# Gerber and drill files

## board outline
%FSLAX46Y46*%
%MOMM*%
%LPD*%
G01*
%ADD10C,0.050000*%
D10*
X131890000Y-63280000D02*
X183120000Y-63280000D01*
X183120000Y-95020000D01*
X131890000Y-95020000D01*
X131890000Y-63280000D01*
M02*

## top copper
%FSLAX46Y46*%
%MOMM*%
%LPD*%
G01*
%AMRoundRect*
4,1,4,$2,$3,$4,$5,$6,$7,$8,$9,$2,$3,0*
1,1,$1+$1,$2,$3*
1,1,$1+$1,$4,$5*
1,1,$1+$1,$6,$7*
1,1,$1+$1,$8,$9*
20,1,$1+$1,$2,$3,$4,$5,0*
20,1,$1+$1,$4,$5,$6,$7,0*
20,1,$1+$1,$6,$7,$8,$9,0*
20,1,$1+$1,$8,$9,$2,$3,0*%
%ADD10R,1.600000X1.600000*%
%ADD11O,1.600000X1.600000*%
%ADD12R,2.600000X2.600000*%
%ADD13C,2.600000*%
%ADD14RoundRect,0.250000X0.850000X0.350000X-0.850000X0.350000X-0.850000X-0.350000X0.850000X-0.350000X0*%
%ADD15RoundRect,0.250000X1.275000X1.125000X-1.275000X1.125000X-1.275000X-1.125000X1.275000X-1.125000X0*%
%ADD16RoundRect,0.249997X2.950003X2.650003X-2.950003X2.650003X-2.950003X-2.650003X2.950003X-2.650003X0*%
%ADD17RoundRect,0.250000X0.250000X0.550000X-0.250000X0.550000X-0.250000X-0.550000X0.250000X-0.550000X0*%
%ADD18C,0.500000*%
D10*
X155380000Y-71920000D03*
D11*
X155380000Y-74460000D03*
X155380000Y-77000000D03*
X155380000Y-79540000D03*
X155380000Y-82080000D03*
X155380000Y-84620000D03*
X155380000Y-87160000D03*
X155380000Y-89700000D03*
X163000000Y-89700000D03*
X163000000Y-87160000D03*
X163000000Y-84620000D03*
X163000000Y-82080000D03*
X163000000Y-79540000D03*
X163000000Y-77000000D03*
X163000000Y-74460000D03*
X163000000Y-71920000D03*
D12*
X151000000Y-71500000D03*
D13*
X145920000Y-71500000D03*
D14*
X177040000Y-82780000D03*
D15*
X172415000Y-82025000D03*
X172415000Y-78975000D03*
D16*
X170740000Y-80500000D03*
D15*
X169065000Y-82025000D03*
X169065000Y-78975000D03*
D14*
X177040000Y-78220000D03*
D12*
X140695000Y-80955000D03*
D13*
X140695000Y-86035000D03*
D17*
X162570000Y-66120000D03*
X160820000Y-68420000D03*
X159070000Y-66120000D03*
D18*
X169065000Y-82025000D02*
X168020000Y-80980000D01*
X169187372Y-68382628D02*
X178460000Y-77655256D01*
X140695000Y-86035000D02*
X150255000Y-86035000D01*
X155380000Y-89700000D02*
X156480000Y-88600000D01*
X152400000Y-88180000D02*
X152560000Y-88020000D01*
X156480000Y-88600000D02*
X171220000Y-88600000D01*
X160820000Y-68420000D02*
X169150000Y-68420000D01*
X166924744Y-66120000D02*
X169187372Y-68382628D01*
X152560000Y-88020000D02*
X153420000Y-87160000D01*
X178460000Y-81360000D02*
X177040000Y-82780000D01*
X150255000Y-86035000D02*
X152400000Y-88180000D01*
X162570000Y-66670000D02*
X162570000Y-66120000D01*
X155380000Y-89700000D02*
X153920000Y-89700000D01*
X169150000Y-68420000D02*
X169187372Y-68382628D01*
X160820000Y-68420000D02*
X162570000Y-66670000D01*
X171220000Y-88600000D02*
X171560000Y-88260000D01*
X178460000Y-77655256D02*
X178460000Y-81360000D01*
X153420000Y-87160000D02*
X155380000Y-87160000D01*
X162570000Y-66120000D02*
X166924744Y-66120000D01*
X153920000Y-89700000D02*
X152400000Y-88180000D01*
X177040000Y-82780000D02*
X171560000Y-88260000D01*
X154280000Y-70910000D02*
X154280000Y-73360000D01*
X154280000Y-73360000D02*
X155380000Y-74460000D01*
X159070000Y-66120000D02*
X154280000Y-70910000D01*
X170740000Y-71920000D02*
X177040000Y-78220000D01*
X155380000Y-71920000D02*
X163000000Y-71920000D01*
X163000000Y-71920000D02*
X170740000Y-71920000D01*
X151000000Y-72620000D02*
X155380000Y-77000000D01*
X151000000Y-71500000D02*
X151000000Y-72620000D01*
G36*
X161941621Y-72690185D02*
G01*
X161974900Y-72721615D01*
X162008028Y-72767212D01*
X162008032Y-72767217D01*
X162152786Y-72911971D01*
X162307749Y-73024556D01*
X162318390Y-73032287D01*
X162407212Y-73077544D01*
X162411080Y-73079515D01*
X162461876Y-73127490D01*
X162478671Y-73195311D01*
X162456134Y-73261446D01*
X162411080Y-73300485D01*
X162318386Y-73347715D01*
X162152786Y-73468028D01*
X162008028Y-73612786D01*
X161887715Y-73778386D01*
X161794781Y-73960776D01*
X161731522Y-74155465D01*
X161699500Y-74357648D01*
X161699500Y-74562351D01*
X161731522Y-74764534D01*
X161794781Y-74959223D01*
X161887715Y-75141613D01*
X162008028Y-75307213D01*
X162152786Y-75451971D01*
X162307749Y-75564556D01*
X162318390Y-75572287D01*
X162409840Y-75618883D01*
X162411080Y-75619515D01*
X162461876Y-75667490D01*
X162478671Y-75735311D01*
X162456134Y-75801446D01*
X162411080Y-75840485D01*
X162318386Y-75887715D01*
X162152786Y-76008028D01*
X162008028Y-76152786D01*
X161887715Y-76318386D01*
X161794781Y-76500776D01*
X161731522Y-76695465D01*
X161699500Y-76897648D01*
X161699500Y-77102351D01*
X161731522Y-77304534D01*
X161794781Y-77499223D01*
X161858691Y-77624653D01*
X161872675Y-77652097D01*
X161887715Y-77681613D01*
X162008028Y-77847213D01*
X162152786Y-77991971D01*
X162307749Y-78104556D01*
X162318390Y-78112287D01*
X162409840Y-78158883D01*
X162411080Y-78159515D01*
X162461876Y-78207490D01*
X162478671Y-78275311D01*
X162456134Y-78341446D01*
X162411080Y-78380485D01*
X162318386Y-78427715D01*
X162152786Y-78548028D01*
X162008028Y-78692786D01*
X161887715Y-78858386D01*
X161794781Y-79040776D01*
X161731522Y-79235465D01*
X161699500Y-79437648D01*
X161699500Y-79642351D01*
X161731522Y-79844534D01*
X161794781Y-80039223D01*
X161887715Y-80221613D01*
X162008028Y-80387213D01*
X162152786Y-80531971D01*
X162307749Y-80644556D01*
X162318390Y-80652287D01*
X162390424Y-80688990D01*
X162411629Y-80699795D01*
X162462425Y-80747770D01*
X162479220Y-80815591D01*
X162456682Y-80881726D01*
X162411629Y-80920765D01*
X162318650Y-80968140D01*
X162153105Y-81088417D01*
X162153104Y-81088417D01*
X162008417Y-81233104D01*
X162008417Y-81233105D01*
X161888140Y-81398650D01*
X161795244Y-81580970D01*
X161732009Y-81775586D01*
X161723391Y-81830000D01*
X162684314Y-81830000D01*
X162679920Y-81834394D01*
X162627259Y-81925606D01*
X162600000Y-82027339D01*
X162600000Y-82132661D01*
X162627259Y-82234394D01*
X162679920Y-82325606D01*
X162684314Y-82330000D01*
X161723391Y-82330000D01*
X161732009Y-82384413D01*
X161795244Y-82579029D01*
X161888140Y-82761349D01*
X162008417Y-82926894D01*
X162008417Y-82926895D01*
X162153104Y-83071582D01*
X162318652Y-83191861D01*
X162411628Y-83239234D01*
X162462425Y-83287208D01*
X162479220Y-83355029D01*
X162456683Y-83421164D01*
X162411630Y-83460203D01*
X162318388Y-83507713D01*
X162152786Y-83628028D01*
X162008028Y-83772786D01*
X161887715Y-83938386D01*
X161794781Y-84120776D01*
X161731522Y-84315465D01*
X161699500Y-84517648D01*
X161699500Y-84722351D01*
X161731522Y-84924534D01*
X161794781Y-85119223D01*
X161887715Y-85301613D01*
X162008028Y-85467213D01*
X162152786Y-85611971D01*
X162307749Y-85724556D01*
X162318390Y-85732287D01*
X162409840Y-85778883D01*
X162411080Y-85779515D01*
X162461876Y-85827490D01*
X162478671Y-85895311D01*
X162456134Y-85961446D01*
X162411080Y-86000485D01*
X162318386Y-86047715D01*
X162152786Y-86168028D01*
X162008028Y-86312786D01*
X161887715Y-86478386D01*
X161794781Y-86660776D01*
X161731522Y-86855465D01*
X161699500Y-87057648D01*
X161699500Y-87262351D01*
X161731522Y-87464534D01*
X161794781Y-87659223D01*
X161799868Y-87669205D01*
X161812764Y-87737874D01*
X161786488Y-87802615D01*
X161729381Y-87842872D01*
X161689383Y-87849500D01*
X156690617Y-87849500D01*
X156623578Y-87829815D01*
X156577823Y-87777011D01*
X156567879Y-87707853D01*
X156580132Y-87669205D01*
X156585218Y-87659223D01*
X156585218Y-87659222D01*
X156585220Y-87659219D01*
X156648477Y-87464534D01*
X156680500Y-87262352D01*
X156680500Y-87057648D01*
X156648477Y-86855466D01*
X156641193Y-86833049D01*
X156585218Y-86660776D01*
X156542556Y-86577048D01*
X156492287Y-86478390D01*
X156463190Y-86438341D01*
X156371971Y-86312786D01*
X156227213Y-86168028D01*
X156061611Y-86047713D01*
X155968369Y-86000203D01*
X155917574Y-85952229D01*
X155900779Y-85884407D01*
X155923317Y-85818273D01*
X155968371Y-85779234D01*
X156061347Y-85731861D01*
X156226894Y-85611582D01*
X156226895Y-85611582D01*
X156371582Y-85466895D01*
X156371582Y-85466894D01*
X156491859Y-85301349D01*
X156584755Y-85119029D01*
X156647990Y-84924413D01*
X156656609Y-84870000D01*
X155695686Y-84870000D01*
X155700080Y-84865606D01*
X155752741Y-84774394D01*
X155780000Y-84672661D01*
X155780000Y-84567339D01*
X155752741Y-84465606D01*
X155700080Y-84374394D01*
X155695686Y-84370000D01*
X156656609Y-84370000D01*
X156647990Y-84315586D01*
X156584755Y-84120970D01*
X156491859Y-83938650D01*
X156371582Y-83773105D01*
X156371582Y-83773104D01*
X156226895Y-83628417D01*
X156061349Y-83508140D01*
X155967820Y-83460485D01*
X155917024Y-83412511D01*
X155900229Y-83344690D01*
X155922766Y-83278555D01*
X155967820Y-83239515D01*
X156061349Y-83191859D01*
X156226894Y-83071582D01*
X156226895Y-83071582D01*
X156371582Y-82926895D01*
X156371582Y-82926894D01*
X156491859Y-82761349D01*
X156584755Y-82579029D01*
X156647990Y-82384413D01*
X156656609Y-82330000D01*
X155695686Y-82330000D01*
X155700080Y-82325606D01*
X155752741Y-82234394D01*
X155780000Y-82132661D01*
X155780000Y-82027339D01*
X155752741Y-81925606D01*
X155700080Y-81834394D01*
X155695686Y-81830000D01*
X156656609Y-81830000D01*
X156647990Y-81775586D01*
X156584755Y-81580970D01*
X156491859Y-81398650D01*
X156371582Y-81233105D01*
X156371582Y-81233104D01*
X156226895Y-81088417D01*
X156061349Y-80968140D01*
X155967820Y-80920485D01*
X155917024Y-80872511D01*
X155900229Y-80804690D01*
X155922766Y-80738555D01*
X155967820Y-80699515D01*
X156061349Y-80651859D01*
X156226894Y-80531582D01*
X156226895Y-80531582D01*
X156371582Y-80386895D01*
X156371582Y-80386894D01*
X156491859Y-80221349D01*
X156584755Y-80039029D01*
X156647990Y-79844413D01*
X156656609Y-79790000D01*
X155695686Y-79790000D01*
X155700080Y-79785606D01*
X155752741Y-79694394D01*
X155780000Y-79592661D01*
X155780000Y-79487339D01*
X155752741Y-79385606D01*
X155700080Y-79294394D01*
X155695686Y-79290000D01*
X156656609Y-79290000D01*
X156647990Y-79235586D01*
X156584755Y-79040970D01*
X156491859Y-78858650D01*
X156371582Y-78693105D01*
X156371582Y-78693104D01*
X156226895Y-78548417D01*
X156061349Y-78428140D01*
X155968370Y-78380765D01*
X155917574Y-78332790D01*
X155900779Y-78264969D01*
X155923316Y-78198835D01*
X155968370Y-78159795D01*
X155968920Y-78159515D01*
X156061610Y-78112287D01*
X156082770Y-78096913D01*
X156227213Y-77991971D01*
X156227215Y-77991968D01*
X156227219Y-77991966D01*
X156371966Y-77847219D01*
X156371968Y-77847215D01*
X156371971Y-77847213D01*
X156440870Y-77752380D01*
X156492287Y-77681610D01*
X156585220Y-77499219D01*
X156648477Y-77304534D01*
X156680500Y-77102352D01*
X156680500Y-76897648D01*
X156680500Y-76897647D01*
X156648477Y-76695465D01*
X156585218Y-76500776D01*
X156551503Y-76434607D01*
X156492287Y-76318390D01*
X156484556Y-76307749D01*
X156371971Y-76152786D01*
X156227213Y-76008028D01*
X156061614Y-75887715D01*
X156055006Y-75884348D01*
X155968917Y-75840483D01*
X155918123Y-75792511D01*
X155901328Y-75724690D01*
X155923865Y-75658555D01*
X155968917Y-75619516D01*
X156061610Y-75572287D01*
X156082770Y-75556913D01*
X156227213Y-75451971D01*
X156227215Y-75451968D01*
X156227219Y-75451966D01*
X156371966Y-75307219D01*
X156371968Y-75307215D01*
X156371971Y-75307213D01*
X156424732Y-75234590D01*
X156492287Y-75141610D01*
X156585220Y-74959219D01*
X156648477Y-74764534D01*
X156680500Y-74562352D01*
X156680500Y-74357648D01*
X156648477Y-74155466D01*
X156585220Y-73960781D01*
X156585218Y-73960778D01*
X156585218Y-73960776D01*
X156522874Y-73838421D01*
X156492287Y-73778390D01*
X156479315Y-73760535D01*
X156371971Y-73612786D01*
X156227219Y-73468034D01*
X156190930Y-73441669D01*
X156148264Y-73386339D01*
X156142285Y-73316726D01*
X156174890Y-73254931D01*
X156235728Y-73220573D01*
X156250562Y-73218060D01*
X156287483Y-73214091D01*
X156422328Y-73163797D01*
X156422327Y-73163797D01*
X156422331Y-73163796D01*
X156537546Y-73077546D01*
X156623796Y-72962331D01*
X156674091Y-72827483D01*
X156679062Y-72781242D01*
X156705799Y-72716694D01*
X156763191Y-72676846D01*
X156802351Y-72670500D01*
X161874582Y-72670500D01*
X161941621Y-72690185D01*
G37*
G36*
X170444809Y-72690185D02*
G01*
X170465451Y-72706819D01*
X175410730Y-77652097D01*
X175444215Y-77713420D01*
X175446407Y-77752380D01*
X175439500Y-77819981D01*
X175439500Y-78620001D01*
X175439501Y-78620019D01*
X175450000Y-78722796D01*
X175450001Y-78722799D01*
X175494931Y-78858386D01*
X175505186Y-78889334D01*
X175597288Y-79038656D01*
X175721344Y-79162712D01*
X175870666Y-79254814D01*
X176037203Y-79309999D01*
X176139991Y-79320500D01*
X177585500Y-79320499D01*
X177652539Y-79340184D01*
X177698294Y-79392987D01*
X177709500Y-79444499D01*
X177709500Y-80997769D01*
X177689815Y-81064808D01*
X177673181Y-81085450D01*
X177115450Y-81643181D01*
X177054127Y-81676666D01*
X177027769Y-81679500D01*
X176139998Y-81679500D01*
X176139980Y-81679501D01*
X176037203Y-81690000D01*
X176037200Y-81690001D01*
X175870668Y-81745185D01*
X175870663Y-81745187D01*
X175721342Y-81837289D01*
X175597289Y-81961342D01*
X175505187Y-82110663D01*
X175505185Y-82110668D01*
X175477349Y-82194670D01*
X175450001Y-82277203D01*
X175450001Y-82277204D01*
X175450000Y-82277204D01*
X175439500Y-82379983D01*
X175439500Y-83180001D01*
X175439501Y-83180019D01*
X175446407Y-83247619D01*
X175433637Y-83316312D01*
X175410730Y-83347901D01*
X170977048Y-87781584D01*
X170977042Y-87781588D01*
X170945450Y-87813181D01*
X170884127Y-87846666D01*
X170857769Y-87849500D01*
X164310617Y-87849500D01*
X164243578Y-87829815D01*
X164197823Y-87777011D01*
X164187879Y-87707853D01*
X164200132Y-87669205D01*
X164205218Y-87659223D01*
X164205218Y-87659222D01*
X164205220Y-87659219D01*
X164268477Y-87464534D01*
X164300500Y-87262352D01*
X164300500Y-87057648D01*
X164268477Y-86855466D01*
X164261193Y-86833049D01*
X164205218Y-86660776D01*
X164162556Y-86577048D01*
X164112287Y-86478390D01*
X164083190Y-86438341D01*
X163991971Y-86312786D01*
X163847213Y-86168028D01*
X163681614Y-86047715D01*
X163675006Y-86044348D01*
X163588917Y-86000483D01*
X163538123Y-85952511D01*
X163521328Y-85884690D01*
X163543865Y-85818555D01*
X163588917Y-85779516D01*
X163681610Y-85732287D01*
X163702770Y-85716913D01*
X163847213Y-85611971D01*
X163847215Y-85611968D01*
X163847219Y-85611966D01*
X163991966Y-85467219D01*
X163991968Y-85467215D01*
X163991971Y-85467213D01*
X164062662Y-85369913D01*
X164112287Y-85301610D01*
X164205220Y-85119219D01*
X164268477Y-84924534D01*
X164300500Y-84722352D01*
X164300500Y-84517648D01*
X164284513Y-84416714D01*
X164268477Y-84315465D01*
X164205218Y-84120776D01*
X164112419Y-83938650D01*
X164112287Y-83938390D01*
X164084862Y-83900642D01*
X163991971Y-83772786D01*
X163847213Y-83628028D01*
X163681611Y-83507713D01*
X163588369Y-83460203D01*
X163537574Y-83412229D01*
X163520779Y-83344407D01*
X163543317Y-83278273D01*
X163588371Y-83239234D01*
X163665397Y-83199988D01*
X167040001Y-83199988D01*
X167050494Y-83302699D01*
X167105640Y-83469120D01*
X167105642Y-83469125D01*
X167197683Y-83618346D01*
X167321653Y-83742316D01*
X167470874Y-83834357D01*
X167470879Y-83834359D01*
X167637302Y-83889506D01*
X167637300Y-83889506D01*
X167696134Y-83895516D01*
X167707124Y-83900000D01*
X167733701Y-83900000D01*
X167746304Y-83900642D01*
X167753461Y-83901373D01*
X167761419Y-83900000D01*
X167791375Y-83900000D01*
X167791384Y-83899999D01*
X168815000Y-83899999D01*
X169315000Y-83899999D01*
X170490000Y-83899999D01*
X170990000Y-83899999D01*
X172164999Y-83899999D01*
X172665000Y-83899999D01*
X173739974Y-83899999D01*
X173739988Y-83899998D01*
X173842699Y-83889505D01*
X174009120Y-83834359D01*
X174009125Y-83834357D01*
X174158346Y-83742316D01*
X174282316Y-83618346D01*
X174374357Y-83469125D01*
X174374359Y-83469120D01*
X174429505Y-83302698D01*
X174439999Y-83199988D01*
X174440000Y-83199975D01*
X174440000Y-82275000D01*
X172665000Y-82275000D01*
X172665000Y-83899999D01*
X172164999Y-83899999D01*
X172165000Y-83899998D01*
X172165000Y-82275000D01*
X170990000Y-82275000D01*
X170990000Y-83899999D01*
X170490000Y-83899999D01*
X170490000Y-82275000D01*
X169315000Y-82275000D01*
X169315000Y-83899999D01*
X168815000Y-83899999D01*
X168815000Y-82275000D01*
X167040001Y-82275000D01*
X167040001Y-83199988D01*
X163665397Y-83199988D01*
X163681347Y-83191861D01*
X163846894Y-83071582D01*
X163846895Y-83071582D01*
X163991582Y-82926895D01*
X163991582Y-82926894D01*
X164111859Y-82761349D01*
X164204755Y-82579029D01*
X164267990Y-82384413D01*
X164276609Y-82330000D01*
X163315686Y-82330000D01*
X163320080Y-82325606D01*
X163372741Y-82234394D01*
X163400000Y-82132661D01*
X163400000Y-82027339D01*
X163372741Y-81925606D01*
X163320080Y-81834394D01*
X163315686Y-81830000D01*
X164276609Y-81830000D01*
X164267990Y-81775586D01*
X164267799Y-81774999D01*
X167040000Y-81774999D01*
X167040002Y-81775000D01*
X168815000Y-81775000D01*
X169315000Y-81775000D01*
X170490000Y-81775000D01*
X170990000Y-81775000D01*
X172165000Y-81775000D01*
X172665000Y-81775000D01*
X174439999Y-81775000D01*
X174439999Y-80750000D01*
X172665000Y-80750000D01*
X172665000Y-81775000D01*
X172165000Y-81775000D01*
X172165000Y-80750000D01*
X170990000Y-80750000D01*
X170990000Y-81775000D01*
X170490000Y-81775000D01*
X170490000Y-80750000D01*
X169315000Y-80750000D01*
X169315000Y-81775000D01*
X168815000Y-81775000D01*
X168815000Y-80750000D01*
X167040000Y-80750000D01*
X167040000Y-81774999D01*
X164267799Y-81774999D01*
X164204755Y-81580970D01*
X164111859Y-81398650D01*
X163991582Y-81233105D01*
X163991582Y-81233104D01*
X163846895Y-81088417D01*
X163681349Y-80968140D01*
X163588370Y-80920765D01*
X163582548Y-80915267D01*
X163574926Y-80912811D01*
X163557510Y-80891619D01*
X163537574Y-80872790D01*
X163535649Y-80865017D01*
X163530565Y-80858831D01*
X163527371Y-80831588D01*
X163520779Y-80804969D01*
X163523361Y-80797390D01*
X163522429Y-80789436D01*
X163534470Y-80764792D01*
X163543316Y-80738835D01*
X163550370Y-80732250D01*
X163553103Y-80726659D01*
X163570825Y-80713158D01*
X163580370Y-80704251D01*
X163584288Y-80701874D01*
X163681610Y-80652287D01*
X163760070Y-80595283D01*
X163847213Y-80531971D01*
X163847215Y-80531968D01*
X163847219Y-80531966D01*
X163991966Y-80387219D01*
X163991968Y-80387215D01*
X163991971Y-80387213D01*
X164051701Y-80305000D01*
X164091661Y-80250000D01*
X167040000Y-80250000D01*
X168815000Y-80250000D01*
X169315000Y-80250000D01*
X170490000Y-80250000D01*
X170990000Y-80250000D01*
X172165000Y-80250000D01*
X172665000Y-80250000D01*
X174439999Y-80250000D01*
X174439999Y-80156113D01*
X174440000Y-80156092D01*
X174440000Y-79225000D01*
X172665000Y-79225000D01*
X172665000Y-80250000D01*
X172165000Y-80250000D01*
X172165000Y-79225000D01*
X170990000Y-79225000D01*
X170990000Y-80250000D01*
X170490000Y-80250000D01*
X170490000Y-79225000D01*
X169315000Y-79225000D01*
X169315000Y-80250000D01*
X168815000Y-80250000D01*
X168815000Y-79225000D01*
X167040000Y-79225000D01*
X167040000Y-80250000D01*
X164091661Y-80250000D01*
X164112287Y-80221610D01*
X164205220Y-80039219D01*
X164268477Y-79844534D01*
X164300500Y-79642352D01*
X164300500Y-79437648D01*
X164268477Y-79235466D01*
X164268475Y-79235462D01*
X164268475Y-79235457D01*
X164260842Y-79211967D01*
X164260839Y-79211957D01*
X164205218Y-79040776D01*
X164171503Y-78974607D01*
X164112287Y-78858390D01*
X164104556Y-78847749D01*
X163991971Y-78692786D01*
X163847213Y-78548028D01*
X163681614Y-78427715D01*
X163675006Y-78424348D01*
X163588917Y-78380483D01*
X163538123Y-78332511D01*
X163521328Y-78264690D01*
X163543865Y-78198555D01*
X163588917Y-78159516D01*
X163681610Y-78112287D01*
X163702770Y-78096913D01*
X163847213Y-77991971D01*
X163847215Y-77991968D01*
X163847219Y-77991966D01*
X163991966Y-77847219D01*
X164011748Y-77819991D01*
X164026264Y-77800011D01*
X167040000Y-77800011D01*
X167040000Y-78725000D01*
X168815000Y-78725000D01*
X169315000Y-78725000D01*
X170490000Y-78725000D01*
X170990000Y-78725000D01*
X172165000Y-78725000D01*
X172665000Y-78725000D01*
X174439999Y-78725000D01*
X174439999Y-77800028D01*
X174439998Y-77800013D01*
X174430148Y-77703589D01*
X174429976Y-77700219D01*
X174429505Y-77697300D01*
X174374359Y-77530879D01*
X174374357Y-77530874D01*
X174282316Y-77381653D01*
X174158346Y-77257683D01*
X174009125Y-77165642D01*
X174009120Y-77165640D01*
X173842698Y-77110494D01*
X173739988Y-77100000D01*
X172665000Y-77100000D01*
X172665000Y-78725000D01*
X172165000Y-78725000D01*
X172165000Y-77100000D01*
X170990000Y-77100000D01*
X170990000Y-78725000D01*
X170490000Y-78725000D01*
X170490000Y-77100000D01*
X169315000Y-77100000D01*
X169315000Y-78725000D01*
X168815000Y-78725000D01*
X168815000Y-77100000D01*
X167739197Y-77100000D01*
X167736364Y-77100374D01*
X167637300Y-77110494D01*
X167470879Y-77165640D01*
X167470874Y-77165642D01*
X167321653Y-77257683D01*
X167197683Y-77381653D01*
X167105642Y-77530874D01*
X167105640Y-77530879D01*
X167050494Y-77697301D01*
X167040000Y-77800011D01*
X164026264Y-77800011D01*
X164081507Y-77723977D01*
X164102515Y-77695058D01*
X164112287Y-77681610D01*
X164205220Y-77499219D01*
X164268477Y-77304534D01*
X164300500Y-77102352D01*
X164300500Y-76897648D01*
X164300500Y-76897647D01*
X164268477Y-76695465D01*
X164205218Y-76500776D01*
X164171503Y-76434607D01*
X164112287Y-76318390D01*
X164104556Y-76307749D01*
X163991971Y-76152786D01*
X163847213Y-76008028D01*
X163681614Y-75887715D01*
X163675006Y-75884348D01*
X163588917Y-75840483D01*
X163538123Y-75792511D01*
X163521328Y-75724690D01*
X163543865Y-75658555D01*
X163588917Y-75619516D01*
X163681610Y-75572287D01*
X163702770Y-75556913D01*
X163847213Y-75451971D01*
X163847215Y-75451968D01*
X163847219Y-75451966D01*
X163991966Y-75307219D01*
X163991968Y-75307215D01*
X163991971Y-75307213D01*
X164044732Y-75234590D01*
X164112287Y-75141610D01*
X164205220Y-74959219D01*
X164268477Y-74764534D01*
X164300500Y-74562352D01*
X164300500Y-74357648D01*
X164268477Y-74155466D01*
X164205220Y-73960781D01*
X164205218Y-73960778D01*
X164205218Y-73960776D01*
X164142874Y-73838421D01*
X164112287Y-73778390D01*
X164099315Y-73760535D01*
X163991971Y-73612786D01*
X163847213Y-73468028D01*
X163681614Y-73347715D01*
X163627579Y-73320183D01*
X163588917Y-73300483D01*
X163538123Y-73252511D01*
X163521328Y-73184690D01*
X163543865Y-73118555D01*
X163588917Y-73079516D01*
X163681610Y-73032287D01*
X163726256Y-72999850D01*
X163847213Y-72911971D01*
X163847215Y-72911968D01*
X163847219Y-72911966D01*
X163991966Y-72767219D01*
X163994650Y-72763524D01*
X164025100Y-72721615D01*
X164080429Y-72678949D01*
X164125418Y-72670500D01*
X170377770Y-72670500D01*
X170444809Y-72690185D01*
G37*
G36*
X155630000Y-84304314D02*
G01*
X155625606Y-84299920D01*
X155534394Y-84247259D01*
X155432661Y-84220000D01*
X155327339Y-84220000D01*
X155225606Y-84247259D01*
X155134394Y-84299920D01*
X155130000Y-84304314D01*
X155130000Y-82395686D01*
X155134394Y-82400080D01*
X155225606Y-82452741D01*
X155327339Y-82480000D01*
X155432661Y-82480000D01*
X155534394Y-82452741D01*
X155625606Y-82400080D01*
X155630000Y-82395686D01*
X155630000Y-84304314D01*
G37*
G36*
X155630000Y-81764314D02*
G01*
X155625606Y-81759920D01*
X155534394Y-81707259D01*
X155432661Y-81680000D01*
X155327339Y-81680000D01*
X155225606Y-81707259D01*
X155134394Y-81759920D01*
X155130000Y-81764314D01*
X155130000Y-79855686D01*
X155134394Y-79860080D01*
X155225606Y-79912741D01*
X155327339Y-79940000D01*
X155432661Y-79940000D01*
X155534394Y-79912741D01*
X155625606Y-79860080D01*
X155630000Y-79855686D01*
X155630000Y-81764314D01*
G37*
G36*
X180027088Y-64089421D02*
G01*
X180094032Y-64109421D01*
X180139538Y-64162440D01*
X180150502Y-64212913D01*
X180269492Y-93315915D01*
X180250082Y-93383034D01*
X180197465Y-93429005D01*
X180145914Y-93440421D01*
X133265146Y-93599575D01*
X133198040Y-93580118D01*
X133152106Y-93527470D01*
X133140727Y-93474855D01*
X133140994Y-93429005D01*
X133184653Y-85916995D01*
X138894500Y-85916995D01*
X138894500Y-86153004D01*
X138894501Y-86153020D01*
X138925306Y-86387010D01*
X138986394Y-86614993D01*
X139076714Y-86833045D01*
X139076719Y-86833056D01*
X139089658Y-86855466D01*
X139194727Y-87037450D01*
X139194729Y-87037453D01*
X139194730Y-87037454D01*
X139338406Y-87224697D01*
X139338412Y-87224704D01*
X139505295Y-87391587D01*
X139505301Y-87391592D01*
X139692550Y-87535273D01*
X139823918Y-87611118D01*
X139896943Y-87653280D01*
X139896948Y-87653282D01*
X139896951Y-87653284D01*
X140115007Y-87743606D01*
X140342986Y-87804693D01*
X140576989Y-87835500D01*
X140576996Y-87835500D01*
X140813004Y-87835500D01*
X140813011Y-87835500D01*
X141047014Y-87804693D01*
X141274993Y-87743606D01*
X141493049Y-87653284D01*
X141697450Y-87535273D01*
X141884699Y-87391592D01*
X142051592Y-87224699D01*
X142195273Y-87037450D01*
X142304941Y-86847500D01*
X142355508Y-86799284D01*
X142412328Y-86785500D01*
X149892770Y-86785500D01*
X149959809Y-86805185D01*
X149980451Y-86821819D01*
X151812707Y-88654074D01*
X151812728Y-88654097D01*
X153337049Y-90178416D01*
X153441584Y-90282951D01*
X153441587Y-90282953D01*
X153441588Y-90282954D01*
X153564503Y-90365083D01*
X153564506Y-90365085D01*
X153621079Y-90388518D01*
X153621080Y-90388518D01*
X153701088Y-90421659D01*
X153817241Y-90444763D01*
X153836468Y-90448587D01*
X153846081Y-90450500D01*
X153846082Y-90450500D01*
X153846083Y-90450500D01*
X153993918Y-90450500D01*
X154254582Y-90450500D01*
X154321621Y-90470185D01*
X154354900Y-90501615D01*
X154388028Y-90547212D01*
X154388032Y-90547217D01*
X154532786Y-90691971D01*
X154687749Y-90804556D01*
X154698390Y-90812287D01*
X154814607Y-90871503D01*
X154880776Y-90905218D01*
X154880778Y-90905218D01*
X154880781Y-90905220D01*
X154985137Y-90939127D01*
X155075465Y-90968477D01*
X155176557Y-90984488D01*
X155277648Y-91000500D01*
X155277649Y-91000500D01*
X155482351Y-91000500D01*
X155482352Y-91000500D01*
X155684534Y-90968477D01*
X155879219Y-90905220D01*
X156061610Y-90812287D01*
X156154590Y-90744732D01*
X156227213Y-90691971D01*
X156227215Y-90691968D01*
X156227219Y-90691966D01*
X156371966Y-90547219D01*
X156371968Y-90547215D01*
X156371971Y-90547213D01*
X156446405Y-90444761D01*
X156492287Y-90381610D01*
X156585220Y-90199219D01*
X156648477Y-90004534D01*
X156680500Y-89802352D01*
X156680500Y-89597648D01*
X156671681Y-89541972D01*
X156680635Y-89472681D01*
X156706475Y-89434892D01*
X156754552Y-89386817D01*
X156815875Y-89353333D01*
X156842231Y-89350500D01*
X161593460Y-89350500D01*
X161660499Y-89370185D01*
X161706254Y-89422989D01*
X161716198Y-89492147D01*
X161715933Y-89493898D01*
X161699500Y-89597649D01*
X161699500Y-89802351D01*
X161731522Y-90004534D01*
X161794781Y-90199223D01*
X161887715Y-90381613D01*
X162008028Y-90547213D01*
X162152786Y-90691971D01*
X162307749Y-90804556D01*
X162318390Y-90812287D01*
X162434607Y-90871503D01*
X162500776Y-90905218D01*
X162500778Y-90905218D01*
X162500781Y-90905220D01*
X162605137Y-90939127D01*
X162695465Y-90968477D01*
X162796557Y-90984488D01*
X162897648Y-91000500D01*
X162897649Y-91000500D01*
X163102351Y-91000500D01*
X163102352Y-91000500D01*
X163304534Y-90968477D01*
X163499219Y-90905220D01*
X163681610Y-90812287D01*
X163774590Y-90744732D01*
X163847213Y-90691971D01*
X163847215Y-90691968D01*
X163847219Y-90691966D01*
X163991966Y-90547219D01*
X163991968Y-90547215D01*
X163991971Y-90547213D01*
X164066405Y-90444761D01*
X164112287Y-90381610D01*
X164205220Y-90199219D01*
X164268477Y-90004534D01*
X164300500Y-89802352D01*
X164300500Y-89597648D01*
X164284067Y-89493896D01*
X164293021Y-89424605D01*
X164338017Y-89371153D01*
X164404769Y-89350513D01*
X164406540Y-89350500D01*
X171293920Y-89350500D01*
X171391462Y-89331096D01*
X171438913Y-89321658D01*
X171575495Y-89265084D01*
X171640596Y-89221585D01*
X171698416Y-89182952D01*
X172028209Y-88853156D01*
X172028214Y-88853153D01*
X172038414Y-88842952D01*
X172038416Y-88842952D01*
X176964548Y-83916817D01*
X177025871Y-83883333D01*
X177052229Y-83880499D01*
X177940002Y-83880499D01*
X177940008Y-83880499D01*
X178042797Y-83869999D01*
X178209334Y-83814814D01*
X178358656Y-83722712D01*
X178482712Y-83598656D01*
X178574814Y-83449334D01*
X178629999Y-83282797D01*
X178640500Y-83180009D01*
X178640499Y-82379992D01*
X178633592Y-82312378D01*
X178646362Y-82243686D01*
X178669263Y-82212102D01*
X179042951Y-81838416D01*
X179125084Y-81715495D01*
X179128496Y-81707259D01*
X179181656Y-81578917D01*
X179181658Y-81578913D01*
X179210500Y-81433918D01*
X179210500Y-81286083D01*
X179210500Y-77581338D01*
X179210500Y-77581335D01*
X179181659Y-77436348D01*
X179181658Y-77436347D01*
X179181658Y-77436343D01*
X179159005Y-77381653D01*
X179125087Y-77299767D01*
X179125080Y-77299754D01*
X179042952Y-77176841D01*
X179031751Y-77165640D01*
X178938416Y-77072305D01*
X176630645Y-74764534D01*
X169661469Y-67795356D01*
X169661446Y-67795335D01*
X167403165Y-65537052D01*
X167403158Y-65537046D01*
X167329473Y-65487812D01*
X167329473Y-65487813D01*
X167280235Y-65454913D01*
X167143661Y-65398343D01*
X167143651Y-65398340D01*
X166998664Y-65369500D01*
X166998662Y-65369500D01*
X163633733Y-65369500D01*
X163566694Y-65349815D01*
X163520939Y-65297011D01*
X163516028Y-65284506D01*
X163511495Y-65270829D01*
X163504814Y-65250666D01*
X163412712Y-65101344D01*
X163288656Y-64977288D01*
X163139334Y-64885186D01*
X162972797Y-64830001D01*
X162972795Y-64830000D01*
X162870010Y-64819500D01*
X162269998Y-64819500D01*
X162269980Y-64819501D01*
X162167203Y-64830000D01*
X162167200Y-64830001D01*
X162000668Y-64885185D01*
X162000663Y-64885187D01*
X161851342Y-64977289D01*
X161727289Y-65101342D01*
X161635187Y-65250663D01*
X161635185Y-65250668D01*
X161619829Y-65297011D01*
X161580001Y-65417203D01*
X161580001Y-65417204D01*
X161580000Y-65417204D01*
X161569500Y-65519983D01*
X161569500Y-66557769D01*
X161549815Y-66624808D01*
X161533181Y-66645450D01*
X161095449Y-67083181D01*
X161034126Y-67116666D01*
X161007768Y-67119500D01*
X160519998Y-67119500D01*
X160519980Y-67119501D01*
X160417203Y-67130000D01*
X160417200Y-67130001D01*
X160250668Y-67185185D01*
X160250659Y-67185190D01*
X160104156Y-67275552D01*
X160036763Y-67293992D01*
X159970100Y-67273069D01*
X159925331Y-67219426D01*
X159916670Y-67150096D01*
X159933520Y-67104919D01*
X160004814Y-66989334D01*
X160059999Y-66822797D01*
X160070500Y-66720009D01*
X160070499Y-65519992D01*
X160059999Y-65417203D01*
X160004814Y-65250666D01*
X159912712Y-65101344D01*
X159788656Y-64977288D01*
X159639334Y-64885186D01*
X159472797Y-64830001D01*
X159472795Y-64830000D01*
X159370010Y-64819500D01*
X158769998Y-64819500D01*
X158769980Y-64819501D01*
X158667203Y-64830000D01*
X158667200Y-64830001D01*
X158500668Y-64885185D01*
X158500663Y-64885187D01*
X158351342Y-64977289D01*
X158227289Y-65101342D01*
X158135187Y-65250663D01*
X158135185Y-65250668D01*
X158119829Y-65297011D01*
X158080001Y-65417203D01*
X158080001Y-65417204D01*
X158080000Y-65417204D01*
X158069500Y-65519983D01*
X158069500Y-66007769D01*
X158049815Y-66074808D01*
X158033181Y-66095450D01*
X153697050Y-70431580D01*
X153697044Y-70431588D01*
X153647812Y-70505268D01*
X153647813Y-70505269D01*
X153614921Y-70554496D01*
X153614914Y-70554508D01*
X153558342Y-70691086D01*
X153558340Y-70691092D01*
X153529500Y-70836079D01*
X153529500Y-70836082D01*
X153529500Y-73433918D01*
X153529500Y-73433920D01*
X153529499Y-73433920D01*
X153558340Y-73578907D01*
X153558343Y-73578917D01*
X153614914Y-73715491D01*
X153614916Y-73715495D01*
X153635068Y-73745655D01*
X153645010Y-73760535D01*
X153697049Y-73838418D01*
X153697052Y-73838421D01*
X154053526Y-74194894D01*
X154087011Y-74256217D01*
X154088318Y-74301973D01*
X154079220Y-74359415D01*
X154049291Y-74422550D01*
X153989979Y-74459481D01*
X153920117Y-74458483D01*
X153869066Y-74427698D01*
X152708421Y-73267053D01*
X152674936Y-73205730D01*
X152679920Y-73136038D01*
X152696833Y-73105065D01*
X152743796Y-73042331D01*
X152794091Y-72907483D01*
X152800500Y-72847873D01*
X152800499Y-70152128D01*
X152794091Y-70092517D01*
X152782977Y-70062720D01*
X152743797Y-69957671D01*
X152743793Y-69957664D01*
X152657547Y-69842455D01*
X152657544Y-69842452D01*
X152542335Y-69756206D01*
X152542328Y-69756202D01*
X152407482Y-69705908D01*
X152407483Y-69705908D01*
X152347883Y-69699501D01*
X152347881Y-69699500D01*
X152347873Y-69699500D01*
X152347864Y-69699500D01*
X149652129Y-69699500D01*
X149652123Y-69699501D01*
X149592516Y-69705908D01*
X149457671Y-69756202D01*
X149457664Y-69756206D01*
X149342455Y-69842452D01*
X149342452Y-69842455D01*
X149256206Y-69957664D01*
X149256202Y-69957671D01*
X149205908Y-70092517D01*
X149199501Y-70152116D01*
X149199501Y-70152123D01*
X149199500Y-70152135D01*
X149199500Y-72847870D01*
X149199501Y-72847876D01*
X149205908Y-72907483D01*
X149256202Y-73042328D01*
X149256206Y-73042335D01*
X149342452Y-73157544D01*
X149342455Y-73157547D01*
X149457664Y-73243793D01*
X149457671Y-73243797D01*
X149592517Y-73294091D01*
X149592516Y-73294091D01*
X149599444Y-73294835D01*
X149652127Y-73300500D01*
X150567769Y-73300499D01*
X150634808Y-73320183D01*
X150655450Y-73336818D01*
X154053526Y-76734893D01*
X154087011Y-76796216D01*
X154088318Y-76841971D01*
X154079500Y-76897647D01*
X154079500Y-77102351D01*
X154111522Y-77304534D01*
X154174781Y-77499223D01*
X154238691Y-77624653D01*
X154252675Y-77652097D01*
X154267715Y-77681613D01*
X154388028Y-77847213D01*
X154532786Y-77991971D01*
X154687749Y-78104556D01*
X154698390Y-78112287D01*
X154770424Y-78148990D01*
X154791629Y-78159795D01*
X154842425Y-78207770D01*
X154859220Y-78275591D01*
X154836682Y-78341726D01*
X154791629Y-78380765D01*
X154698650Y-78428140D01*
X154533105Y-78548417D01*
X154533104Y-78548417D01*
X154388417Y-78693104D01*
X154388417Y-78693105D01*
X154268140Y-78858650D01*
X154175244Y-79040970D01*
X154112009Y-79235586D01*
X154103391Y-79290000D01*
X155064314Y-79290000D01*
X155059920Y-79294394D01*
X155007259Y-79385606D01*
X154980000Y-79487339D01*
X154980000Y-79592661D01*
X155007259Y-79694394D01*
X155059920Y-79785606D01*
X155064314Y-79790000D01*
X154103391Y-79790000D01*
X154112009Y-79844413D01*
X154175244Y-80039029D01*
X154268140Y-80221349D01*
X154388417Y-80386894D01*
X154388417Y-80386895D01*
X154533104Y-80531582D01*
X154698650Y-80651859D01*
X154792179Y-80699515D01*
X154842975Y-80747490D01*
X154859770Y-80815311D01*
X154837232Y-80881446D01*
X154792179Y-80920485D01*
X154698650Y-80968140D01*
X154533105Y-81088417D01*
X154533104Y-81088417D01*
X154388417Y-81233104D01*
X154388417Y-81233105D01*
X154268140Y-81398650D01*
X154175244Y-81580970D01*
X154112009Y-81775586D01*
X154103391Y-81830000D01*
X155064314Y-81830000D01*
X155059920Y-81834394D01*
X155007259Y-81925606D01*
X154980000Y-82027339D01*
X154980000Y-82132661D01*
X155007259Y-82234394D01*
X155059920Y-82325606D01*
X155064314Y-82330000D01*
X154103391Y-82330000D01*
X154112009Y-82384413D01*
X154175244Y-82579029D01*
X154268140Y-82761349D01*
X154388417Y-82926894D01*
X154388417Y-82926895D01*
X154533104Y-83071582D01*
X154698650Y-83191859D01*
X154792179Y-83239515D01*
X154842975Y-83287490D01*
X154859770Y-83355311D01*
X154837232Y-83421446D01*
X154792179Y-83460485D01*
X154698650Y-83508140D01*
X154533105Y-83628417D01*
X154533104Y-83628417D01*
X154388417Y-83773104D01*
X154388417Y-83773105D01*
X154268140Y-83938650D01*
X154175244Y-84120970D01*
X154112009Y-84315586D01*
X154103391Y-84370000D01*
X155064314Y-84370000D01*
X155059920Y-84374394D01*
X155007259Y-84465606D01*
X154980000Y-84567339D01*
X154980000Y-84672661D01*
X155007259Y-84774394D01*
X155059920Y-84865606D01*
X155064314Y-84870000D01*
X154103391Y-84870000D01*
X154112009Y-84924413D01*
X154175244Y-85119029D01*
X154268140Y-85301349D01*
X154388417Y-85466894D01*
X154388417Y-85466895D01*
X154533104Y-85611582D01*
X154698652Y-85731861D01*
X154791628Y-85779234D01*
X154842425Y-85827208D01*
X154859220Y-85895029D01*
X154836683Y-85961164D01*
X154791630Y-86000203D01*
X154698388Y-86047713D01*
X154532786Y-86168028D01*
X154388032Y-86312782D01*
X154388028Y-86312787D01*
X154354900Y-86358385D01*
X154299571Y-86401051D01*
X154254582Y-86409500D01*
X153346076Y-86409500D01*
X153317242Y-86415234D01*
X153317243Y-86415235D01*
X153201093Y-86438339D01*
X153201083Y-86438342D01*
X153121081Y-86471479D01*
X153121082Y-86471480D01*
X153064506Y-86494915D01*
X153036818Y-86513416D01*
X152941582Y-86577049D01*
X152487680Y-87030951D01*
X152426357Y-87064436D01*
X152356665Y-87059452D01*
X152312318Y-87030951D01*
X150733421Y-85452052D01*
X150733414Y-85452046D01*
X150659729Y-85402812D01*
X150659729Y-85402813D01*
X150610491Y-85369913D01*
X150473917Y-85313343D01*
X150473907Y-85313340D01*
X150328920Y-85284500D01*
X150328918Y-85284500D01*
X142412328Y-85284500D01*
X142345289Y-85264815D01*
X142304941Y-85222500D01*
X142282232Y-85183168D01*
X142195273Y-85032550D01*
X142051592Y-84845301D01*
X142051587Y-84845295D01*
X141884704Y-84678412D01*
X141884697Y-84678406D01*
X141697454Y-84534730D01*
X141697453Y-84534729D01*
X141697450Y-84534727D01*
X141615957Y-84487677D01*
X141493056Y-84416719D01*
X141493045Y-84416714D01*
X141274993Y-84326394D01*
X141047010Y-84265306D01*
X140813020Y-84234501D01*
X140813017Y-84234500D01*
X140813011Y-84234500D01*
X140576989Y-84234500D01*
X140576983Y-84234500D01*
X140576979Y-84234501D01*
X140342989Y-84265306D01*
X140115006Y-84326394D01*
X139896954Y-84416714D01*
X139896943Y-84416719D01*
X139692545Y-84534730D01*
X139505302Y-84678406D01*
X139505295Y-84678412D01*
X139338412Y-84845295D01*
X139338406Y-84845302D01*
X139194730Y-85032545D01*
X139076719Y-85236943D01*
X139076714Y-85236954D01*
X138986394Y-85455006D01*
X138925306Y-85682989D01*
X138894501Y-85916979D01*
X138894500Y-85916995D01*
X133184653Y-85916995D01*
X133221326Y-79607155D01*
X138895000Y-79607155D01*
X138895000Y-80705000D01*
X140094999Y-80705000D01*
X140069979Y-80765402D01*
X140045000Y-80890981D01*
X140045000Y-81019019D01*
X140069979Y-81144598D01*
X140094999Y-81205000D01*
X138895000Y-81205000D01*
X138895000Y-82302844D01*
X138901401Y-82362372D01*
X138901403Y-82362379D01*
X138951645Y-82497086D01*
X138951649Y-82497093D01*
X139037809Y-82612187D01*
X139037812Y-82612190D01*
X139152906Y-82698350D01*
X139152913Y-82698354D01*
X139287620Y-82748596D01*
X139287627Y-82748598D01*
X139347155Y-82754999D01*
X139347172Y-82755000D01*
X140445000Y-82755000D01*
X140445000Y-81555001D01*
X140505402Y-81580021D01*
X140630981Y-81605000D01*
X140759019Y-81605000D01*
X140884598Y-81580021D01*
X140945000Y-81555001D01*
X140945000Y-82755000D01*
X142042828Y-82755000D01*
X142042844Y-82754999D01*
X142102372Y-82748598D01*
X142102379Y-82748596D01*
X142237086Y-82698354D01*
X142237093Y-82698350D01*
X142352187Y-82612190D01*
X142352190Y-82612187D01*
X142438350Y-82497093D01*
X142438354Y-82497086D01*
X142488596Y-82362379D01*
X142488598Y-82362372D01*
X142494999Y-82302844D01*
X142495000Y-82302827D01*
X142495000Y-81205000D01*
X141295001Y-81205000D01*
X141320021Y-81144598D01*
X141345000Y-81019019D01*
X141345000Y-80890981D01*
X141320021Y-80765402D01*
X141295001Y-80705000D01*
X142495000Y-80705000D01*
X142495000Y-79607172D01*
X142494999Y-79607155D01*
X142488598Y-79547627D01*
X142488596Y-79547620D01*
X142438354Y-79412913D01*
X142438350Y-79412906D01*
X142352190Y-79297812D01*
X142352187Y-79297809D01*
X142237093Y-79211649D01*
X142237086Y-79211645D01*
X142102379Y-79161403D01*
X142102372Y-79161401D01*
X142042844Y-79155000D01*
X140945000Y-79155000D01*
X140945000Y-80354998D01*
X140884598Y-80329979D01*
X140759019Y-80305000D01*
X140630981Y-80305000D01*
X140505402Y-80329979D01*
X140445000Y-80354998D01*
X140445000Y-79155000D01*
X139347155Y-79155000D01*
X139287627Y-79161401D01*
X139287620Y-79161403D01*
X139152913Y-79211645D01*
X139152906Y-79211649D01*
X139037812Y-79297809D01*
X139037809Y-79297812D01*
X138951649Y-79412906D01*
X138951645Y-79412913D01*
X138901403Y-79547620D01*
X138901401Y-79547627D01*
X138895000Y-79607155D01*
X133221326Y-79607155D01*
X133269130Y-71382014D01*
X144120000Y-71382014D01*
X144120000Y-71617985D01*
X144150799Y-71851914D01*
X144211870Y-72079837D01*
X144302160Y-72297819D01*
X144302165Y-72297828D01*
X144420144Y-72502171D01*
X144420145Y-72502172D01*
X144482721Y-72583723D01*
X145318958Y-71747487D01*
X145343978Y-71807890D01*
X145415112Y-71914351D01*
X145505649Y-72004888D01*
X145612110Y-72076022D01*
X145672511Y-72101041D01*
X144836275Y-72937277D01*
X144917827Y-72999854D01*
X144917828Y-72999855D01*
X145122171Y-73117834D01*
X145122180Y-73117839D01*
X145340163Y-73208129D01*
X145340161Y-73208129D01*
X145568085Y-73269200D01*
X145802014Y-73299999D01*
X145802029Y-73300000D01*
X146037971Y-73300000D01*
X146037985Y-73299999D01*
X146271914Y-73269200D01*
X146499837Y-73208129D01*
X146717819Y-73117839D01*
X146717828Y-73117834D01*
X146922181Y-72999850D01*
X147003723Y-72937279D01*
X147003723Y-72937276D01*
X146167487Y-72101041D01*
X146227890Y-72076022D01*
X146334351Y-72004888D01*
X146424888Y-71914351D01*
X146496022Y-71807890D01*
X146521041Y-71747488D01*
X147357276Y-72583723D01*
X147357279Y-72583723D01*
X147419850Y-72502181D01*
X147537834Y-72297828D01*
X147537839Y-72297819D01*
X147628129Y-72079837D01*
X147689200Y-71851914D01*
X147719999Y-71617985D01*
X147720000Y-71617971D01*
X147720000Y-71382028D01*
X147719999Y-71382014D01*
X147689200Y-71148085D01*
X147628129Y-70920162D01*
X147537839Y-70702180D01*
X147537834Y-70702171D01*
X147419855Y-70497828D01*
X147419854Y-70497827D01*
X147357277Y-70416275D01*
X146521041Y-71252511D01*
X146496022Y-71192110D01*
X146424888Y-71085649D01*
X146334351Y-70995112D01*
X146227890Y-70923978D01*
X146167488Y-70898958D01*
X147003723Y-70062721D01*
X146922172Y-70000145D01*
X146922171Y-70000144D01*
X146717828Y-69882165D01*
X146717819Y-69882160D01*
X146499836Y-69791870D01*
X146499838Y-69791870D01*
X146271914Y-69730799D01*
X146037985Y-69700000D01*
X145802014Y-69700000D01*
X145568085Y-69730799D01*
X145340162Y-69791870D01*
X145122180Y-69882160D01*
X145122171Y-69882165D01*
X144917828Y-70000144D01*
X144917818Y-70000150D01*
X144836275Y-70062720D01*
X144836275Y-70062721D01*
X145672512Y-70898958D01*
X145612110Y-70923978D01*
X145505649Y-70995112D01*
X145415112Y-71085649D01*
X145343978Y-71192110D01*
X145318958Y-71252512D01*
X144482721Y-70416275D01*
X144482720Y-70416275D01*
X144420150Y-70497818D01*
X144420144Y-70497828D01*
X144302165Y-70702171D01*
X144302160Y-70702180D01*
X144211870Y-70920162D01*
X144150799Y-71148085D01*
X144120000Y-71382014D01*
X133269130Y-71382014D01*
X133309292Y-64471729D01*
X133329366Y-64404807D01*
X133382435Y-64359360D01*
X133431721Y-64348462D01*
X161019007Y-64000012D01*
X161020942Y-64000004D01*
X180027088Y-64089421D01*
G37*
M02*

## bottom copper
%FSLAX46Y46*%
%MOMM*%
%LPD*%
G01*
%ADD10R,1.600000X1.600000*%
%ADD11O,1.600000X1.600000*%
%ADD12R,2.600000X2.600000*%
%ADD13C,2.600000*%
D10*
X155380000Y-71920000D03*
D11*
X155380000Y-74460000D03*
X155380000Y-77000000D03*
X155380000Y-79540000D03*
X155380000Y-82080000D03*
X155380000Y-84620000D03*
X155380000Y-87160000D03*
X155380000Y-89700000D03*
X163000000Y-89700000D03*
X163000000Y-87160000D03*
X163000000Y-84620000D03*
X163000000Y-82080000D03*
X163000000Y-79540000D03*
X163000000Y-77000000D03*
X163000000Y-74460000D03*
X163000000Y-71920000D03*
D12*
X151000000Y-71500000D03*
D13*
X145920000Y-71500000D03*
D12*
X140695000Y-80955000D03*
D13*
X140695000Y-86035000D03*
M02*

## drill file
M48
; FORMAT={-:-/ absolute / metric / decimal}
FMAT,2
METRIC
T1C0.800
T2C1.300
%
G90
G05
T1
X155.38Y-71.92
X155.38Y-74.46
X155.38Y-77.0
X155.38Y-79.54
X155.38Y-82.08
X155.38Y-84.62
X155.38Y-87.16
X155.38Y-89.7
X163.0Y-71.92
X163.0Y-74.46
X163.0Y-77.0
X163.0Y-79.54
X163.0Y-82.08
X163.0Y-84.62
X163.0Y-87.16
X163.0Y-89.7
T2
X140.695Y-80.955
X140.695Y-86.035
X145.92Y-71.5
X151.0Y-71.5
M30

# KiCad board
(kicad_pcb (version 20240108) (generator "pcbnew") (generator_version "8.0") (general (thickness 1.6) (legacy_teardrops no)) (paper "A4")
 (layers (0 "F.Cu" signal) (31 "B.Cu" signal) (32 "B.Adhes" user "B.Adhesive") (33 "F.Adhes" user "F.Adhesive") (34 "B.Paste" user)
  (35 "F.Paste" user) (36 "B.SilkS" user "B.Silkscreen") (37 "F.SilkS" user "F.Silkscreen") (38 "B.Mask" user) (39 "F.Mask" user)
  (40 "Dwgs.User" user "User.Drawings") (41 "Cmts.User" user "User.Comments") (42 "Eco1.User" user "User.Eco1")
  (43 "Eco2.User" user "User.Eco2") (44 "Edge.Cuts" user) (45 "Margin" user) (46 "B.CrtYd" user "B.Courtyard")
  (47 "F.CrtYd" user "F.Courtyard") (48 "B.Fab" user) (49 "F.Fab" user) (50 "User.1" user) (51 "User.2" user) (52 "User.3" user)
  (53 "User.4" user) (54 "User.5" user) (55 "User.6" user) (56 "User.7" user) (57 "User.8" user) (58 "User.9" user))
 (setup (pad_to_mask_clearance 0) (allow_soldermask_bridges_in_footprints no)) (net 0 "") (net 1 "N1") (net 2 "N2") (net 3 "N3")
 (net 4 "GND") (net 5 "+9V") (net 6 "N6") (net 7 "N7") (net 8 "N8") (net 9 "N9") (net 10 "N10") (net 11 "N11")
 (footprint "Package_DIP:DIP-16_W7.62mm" (layer "F.Cu") (at 155.38 71.92)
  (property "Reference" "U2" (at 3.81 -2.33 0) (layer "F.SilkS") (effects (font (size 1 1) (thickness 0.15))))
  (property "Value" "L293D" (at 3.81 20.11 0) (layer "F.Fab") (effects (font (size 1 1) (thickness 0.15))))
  (pad "1" thru_hole rect (at 0 0) (size 1.6 1.6) (drill 0.8) (layers "*.Cu" "*.Mask") (remove_unused_layers no) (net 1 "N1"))
  (pad "2" thru_hole oval (at 0 2.54) (size 1.6 1.6) (drill 0.8) (layers "*.Cu" "*.Mask") (remove_unused_layers no) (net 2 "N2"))
  (pad "3" thru_hole oval (at 0 5.08) (size 1.6 1.6) (drill 0.8) (layers "*.Cu" "*.Mask") (remove_unused_layers no) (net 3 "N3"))
  (pad "4" thru_hole oval (at 0 7.62) (size 1.6 1.6) (drill 0.8) (layers "*.Cu" "*.Mask") (remove_unused_layers no) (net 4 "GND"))
  (pad "5" thru_hole oval (at 0 10.16) (size 1.6 1.6) (drill 0.8) (layers "*.Cu" "*.Mask") (remove_unused_layers no) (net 4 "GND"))
  (pad "6" thru_hole oval (at 0 12.7) (size 1.6 1.6) (drill 0.8) (layers "*.Cu" "*.Mask") (remove_unused_layers no) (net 4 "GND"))
  (pad "7" thru_hole oval (at 0 15.24) (size 1.6 1.6) (drill 0.8) (layers "*.Cu" "*.Mask") (remove_unused_layers no) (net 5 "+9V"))
  (pad "8" thru_hole oval (at 0 17.78) (size 1.6 1.6) (drill 0.8) (layers "*.Cu" "*.Mask") (remove_unused_layers no) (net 5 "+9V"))
  (pad "9" thru_hole oval (at 7.62 17.78) (size 1.6 1.6) (drill 0.8) (layers "*.Cu" "*.Mask") (remove_unused_layers no) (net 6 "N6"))
  (pad "10" thru_hole oval (at 7.62 15.24) (size 1.6 1.6) (drill 0.8) (layers "*.Cu" "*.Mask") (remove_unused_layers no) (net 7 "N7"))
  (pad "11" thru_hole oval (at 7.62 12.7) (size 1.6 1.6) (drill 0.8) (layers "*.Cu" "*.Mask") (remove_unused_layers no) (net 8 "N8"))
  (pad "12" thru_hole oval (at 7.62 10.16) (size 1.6 1.6) (drill 0.8) (layers "*.Cu" "*.Mask") (remove_unused_layers no) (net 4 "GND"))
  (pad "13" thru_hole oval (at 7.62 7.62) (size 1.6 1.6) (drill 0.8) (layers "*.Cu" "*.Mask") (remove_unused_layers no) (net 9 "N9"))
  (pad "14" thru_hole oval (at 7.62 5.08) (size 1.6 1.6) (drill 0.8) (layers "*.Cu" "*.Mask") (remove_unused_layers no) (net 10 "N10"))
  (pad "15" thru_hole oval (at 7.62 2.54) (size 1.6 1.6) (drill 0.8) (layers "*.Cu" "*.Mask") (remove_unused_layers no) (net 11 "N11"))
  (pad "16" thru_hole oval (at 7.62 0) (size 1.6 1.6) (drill 0.8) (layers "*.Cu" "*.Mask") (remove_unused_layers no) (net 1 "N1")))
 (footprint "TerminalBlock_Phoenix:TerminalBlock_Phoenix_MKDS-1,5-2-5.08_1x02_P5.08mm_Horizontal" (layer "F.Cu") (at 151 71.5 180)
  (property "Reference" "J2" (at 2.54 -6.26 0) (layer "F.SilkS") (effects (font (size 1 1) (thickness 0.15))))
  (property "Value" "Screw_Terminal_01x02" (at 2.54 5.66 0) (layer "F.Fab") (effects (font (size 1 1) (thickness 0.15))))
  (pad "1" thru_hole rect (at 0 0 180) (size 2.6 2.6) (drill 1.3) (layers "*.Cu" "*.Mask") (remove_unused_layers no) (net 3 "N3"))
  (pad "2" thru_hole circle (at 5.08 0 180) (size 2.6 2.6) (drill 1.3) (layers "*.Cu" "*.Mask") (remove_unused_layers no) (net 4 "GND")))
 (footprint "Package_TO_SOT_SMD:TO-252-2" (layer "F.Cu") (at 172 80.5 180)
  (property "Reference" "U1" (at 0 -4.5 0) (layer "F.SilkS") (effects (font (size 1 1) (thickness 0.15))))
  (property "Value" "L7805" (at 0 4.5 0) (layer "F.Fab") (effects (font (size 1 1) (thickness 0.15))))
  (pad "1" smd roundrect (at -5.04 -2.28 180) (size 2.2 1.2) (layers "F.Cu" "F.Paste" "F.Mask") (roundrect_rratio 0.208333) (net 5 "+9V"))
  (pad "2" smd roundrect (at -0.415 -1.525 180) (size 3.05 2.75) (layers "F.Cu" "F.Paste") (roundrect_rratio 0.090909) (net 4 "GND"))
  (pad "2" smd roundrect (at -0.415 1.525 180) (size 3.05 2.75) (layers "F.Cu" "F.Paste") (roundrect_rratio 0.090909) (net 4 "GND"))
  (pad "2" smd roundrect (at 1.26 0 180) (size 6.4 5.8) (layers "F.Cu" "F.Mask") (roundrect_rratio 0.043103) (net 4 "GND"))
  (pad "2" smd roundrect (at 2.935 -1.525 180) (size 3.05 2.75) (layers "F.Cu" "F.Paste") (roundrect_rratio 0.090909) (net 4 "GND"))
  (pad "2" smd roundrect (at 2.935 1.525 180) (size 3.05 2.75) (layers "F.Cu" "F.Paste") (roundrect_rratio 0.090909) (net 4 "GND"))
  (pad "3" smd roundrect (at -5.04 2.28 180) (size 2.2 1.2) (layers "F.Cu" "F.Paste" "F.Mask") (roundrect_rratio 0.208333) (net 1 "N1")))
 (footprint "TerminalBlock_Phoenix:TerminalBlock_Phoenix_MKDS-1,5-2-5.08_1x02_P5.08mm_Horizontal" (layer "F.Cu") (at 140.695 80.955 -90)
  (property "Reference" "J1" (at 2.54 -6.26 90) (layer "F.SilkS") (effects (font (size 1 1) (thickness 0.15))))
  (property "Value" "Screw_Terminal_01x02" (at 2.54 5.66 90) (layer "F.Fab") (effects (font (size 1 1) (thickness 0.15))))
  (pad "1" thru_hole rect (at 0 0 270) (size 2.6 2.6) (drill 1.3) (layers "*.Cu" "*.Mask") (remove_unused_layers no) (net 4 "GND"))
  (pad "2" thru_hole circle (at 5.08 0 270) (size 2.6 2.6) (drill 1.3) (layers "*.Cu" "*.Mask") (remove_unused_layers no) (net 5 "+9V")))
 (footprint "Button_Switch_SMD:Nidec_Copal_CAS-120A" (layer "F.Cu") (at 160.82 67.27 -90)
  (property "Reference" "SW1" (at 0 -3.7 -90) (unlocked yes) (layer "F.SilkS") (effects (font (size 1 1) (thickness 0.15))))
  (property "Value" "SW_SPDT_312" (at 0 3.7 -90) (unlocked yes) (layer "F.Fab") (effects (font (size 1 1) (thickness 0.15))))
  (pad "1" smd roundrect (at -1.15 -1.75 180) (size 1 1.6) (layers "F.Cu" "F.Paste" "F.Mask") (roundrect_rratio 0.25) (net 5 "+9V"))
  (pad "2" smd roundrect (at 1.15 0 180) (size 1 1.6) (layers "F.Cu" "F.Paste" "F.Mask") (roundrect_rratio 0.25) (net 5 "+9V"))
  (pad "3" smd roundrect (at -1.15 1.75 180) (size 1 1.6) (layers "F.Cu" "F.Paste" "F.Mask") (roundrect_rratio 0.25) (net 2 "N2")))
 (gr_rect (start 131.89 63.28) (end 183.12 95.02) (stroke (width 0.05) (type default)) (fill none) (layer "Edge.Cuts"))
 (segment (start 169.065 82.025) (end 168.02 80.98) (width 0.5) (layer "F.Cu") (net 4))
 (segment (start 169.187372 68.382628) (end 178.46 77.655256) (width 0.5) (layer "F.Cu") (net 5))
 (segment (start 140.695 86.035) (end 150.255 86.035) (width 0.5) (layer "F.Cu") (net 5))
 (segment (start 155.38 89.7) (end 156.48 88.6) (width 0.5) (layer "F.Cu") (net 5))
 (segment (start 152.4 88.18) (end 152.56 88.02) (width 0.5) (layer "F.Cu") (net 5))
 (segment (start 156.48 88.6) (end 171.22 88.6) (width 0.5) (layer "F.Cu") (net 5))
 (segment (start 160.82 68.42) (end 169.15 68.42) (width 0.5) (layer "F.Cu") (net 5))
 (segment (start 166.924744 66.12) (end 169.187372 68.382628) (width 0.5) (layer "F.Cu") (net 5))
 (segment (start 152.56 88.02) (end 153.42 87.16) (width 0.5) (layer "F.Cu") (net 5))
 (segment (start 178.46 81.36) (end 177.04 82.78) (width 0.5) (layer "F.Cu") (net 5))
 (segment (start 150.255 86.035) (end 152.4 88.18) (width 0.5) (layer "F.Cu") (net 5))
 (segment (start 162.57 66.67) (end 162.57 66.12) (width 0.5) (layer "F.Cu") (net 5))
 (segment (start 155.38 89.7) (end 153.92 89.7) (width 0.5) (layer "F.Cu") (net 5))
 (segment (start 169.15 68.42) (end 169.187372 68.382628) (width 0.5) (layer "F.Cu") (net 5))
 (segment (start 160.82 68.42) (end 162.57 66.67) (width 0.5) (layer "F.Cu") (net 5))
 (segment (start 171.22 88.6) (end 171.56 88.26) (width 0.5) (layer "F.Cu") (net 5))
 (segment (start 178.46 77.655256) (end 178.46 81.36) (width 0.5) (layer "F.Cu") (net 5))
 (segment (start 153.42 87.16) (end 155.38 87.16) (width 0.5) (layer "F.Cu") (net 5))
 (segment (start 162.57 66.12) (end 166.924744 66.12) (width 0.5) (layer "F.Cu") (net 5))
 (segment (start 153.92 89.7) (end 152.4 88.18) (width 0.5) (layer "F.Cu") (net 5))
 (segment (start 177.04 82.78) (end 171.56 88.26) (width 0.5) (layer "F.Cu") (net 5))
 (segment (start 154.28 70.91) (end 154.28 73.36) (width 0.5) (layer "F.Cu") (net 2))
 (segment (start 154.28 73.36) (end 155.38 74.46) (width 0.5) (layer "F.Cu") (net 2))
 (segment (start 159.07 66.12) (end 154.28 70.91) (width 0.5) (layer "F.Cu") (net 2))
 (segment (start 170.74 71.92) (end 177.04 78.22) (width 0.5) (layer "F.Cu") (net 1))
 (segment (start 155.38 71.92) (end 163 71.92) (width 0.5) (layer "F.Cu") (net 1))
 (segment (start 163 71.92) (end 170.74 71.92) (width 0.5) (layer "F.Cu") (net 1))
 (segment (start 151 72.62) (end 155.38 77) (width 0.5) (layer "F.Cu") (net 3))
 (segment (start 151 71.5) (end 151 72.62) (width 0.5) (layer "F.Cu") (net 3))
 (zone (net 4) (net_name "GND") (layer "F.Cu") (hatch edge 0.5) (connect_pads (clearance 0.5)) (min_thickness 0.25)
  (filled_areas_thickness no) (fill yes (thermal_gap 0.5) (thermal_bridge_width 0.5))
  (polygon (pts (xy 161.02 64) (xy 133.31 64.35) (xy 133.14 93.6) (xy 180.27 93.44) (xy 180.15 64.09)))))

